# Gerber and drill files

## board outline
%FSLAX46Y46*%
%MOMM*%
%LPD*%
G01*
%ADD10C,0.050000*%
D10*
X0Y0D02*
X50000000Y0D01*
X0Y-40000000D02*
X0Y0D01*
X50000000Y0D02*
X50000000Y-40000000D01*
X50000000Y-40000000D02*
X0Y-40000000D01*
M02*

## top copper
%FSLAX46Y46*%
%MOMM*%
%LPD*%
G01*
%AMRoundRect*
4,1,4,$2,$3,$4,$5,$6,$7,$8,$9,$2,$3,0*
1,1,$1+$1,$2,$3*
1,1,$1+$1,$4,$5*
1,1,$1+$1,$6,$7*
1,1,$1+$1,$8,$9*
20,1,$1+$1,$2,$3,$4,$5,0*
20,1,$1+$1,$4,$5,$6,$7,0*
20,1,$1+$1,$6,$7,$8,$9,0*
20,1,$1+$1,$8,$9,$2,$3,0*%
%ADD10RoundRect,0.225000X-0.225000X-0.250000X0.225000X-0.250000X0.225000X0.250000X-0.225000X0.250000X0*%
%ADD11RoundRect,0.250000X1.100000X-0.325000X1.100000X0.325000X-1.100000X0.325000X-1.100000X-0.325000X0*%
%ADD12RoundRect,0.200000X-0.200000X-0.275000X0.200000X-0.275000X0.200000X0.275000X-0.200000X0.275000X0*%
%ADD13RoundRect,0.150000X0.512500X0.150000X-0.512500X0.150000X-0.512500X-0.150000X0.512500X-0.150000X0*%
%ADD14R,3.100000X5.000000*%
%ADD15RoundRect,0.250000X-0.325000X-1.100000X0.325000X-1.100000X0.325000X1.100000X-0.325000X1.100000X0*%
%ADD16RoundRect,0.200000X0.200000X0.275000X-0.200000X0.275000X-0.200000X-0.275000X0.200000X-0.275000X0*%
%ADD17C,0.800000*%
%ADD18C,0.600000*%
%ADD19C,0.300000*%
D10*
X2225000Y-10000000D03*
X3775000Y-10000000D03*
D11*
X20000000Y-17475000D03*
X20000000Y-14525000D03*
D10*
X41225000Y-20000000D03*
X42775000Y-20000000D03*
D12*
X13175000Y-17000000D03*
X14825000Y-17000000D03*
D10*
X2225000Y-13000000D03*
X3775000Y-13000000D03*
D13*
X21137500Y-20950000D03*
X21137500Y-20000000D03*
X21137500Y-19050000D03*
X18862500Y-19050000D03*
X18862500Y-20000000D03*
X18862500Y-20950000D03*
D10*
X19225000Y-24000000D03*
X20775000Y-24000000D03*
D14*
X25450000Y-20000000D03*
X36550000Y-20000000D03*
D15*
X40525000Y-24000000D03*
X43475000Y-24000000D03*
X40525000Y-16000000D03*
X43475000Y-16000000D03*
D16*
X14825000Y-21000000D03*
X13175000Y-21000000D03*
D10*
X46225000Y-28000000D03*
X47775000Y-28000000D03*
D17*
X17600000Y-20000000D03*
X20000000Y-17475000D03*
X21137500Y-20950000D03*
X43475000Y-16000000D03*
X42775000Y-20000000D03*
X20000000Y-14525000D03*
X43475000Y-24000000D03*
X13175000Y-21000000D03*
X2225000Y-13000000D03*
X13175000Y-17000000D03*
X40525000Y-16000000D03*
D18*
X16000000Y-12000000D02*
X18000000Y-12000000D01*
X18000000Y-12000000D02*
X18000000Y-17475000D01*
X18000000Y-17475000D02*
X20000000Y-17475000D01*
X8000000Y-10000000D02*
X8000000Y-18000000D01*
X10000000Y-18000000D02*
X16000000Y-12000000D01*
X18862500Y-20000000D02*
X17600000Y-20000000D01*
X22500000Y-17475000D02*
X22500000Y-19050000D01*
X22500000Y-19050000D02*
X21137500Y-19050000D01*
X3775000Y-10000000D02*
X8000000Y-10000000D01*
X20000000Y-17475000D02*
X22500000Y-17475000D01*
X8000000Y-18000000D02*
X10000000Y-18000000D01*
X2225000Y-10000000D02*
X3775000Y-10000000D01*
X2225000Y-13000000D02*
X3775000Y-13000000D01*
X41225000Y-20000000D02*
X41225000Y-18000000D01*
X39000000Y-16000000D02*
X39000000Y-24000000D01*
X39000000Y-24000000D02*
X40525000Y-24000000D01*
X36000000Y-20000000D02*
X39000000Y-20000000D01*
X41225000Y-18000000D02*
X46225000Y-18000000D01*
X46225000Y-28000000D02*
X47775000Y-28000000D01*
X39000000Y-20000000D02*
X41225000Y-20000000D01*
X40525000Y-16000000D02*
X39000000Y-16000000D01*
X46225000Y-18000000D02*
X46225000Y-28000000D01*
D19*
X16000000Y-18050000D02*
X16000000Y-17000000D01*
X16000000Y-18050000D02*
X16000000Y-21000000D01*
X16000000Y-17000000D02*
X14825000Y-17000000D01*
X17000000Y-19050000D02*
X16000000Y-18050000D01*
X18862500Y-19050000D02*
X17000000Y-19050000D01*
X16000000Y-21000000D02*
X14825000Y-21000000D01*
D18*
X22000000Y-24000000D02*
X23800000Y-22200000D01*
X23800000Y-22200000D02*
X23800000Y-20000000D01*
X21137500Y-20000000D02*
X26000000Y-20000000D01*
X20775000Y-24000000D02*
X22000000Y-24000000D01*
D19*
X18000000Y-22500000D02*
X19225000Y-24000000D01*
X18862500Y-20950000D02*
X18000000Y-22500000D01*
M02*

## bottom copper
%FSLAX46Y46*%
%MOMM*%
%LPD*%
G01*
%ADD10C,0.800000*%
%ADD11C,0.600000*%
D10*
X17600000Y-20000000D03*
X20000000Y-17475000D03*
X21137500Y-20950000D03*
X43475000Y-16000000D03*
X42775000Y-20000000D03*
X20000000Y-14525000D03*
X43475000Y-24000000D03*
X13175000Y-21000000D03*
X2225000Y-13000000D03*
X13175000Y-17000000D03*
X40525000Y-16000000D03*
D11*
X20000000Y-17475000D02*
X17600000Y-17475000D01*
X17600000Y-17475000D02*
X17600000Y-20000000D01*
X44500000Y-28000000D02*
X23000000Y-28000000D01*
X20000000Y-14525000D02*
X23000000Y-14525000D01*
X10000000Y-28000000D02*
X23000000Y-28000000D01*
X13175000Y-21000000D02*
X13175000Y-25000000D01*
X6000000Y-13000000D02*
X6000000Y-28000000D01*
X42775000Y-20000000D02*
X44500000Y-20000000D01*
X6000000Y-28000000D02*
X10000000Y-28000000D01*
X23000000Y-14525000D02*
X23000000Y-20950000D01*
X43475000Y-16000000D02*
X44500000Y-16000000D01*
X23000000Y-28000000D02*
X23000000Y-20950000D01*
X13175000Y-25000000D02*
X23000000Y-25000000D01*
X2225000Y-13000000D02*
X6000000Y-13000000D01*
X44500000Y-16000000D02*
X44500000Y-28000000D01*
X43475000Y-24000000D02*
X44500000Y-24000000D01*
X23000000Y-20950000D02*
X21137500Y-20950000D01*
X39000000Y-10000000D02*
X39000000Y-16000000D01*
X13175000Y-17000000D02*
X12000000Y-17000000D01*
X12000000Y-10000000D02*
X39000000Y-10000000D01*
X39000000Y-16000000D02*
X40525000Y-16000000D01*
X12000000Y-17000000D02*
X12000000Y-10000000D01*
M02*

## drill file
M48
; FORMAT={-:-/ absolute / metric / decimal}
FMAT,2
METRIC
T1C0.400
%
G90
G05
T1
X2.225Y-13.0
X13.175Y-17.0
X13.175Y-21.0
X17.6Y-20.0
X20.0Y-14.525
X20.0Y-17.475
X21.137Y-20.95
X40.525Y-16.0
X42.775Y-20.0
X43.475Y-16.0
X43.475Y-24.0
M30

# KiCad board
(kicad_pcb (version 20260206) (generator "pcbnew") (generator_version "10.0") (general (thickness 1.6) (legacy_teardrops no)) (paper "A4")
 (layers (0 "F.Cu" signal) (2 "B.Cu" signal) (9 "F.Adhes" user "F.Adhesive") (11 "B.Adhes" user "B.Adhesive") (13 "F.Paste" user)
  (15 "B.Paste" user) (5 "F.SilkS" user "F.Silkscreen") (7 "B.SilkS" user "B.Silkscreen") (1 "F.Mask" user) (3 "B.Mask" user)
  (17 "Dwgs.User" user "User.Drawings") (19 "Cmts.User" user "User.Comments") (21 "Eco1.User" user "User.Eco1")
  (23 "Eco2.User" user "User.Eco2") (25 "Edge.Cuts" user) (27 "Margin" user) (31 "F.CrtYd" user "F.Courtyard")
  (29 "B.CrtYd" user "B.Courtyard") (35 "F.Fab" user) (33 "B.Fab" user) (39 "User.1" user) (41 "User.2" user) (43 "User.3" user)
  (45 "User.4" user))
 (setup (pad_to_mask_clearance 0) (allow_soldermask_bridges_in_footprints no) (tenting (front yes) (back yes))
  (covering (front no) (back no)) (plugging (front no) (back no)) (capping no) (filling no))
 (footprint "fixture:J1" (layer "F.Cu") (at 3 10)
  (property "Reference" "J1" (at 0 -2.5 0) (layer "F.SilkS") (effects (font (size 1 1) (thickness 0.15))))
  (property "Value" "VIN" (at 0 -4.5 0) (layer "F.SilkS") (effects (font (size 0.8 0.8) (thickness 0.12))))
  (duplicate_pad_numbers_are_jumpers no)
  (pad "1" smd roundrect (at -0.775 0) (size 0.9 0.95) (layers "F.Cu" "F.Mask" "F.Paste") (roundrect_rratio 0.25) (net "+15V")
   (thermal_bridge_angle 45))
  (pad "2" smd roundrect (at 0.775 0) (size 0.9 0.95) (layers "F.Cu" "F.Mask" "F.Paste") (roundrect_rratio 0.25) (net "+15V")
   (thermal_bridge_angle 45)))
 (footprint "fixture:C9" (layer "F.Cu") (at 20 16 90)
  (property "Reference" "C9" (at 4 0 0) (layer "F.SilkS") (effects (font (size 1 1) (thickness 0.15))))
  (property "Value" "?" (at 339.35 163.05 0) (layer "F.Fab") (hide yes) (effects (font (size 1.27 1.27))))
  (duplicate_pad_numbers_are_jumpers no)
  (pad "1" smd roundrect (at -1.475 0 90) (size 1.15 2.7) (layers "F.Cu" "F.Mask" "F.Paste") (roundrect_rratio 0.217391) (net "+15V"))
  (pad "2" smd roundrect (at 1.475 0 90) (size 1.15 2.7) (layers "F.Cu" "F.Mask" "F.Paste") (roundrect_rratio 0.217391) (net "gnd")))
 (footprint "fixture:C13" (layer "F.Cu") (at 42 20)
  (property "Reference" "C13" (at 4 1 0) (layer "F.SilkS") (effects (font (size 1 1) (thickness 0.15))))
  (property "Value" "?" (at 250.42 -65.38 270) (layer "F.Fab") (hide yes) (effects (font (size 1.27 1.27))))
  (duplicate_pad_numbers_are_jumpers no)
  (pad "1" smd roundrect (at -0.775 0) (size 0.9 0.95) (layers "F.Cu" "F.Mask" "F.Paste") (roundrect_rratio 0.25) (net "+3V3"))
  (pad "2" smd roundrect (at 0.775 0) (size 0.9 0.95) (layers "F.Cu" "F.Mask" "F.Paste") (roundrect_rratio 0.25) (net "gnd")))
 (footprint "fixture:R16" (layer "F.Cu") (at 14 17)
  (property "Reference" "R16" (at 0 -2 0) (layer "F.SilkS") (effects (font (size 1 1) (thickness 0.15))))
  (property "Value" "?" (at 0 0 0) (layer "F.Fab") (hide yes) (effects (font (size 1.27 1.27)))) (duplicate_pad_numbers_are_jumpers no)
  (pad "1" smd roundrect (at -0.825 0) (size 0.8 0.95) (layers "F.Cu" "F.Mask" "F.Paste") (roundrect_rratio 0.25) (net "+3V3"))
  (pad "2" smd roundrect (at 0.825 0) (size 0.8 0.95) (layers "F.Cu" "F.Mask" "F.Paste") (roundrect_rratio 0.25) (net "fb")))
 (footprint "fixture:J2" (layer "F.Cu") (at 3 13)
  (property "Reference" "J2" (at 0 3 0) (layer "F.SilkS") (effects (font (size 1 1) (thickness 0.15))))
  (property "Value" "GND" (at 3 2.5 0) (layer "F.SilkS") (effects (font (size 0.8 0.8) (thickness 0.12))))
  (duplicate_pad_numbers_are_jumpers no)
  (pad "1" smd roundrect (at -0.775 0) (size 0.9 0.95) (layers "F.Cu" "F.Mask" "F.Paste") (roundrect_rratio 0.25) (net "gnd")
   (thermal_bridge_angle 45))
  (pad "2" smd roundrect (at 0.775 0) (size 0.9 0.95) (layers "F.Cu" "F.Mask" "F.Paste") (roundrect_rratio 0.25) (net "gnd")
   (thermal_bridge_angle 45)))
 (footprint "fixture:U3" (layer "F.Cu") (at 20 20 180)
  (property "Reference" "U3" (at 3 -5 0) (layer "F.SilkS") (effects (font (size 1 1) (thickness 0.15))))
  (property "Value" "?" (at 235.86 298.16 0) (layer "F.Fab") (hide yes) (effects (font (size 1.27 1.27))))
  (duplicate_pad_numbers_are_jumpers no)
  (pad "1" smd roundrect (at -1.1375 -0.95 180) (size 1.325 0.6) (layers "F.Cu" "F.Mask" "F.Paste") (roundrect_rratio 0.25) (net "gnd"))
  (pad "2" smd roundrect (at -1.1375 0 180) (size 1.325 0.6) (layers "F.Cu" "F.Mask" "F.Paste") (roundrect_rratio 0.25) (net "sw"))
  (pad "3" smd roundrect (at -1.1375 0.95 180) (size 1.325 0.6) (layers "F.Cu" "F.Mask" "F.Paste") (roundrect_rratio 0.25) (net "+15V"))
  (pad "4" smd roundrect (at 1.1375 0.95 180) (size 1.325 0.6) (layers "F.Cu" "F.Mask" "F.Paste") (roundrect_rratio 0.25) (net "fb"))
  (pad "5" smd roundrect (at 1.1375 0 180) (size 1.325 0.6) (layers "F.Cu" "F.Mask" "F.Paste") (roundrect_rratio 0.25) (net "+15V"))
  (pad "6" smd roundrect (at 1.1375 -0.95 180) (size 1.325 0.6) (layers "F.Cu" "F.Mask" "F.Paste") (roundrect_rratio 0.25) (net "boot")))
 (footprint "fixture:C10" (layer "F.Cu") (at 20 24)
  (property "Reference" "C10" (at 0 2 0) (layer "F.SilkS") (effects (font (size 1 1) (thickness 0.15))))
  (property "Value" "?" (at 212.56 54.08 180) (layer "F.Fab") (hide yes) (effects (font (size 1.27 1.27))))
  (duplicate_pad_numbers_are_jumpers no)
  (pad "1" smd roundrect (at -0.775 0) (size 0.9 0.95) (layers "F.Cu" "F.Mask" "F.Paste") (roundrect_rratio 0.25) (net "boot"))
  (pad "2" smd roundrect (at 0.775 0) (size 0.9 0.95) (layers "F.Cu" "F.Mask" "F.Paste") (roundrect_rratio 0.25) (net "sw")))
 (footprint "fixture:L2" (layer "F.Cu") (at 31 20)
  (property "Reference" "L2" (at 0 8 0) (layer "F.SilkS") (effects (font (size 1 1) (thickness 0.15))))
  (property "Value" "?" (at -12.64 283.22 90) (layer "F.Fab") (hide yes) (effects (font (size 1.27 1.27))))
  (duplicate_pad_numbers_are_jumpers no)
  (pad "1" smd rect (at -5.55 0) (size 3.1 5) (layers "F.Cu" "F.Mask" "F.Paste") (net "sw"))
  (pad "2" smd rect (at 5.55 0) (size 3.1 5) (layers "F.Cu" "F.Mask" "F.Paste") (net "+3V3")))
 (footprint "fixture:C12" (layer "F.Cu") (at 42 24)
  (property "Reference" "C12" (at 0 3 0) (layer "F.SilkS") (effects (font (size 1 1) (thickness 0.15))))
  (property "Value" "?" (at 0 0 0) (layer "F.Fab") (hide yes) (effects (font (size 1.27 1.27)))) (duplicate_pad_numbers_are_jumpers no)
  (pad "1" smd roundrect (at -1.475 0) (size 1.15 2.7) (layers "F.Cu" "F.Mask" "F.Paste") (roundrect_rratio 0.217391) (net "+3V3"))
  (pad "2" smd roundrect (at 1.475 0) (size 1.15 2.7) (layers "F.Cu" "F.Mask" "F.Paste") (roundrect_rratio 0.217391) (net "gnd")))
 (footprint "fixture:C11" (layer "F.Cu") (at 42 16)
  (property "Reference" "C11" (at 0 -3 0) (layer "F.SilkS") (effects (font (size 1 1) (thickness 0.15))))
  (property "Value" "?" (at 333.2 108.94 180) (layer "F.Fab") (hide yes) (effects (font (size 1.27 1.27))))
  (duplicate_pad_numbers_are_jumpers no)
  (pad "1" smd roundrect (at -1.475 0) (size 1.15 2.7) (layers "F.Cu" "F.Mask" "F.Paste") (roundrect_rratio 0.217391) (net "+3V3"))
  (pad "2" smd roundrect (at 1.475 0) (size 1.15 2.7) (layers "F.Cu" "F.Mask" "F.Paste") (roundrect_rratio 0.217391) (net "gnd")))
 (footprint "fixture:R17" (layer "F.Cu") (at 14 21 180)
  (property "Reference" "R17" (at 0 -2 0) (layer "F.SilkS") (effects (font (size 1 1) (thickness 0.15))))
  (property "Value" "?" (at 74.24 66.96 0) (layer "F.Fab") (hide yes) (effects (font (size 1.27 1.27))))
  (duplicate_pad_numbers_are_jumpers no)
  (pad "1" smd roundrect (at -0.825 0 180) (size 0.8 0.95) (layers "F.Cu" "F.Mask" "F.Paste") (roundrect_rratio 0.25) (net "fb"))
  (pad "2" smd roundrect (at 0.825 0 180) (size 0.8 0.95) (layers "F.Cu" "F.Mask" "F.Paste") (roundrect_rratio 0.25) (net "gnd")))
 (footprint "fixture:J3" (layer "F.Cu") (at 47 28)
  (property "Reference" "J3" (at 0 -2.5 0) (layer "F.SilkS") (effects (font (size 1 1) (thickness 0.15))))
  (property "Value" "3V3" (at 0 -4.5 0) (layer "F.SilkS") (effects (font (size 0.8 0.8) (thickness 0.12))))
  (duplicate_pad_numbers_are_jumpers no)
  (pad "1" smd roundrect (at -0.775 0) (size 0.9 0.95) (layers "F.Cu" "F.Mask" "F.Paste") (roundrect_rratio 0.25) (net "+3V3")
   (thermal_bridge_angle 45))
  (pad "2" smd roundrect (at 0.775 0) (size 0.9 0.95) (layers "F.Cu" "F.Mask" "F.Paste") (roundrect_rratio 0.25) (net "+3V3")
   (thermal_bridge_angle 45)))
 (gr_line (start 0 0) (end 50 0) (stroke (width 0.05) (type default)) (layer "Edge.Cuts"))
 (gr_line (start 0 40) (end 0 0) (stroke (width 0.05) (type default)) (layer "Edge.Cuts"))
 (gr_line (start 50 0) (end 50 40) (stroke (width 0.05) (type default)) (layer "Edge.Cuts"))
 (gr_line (start 50 40) (end 0 40) (stroke (width 0.05) (type default)) (layer "Edge.Cuts"))
 (segment (start 16 12) (end 18 12) (width 0.6) (layer "F.Cu") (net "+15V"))
 (segment (start 18 12) (end 18 17.475) (width 0.6) (layer "F.Cu") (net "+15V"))
 (segment (start 18 17.475) (end 20 17.475) (width 0.6) (layer "F.Cu") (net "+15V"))
 (segment (start 8 10) (end 8 18) (width 0.6) (layer "F.Cu") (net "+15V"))
 (segment (start 10 18) (end 16 12) (width 0.6) (layer "F.Cu") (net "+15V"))
 (segment (start 18.8625 20) (end 17.6 20) (width 0.6) (layer "F.Cu") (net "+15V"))
 (segment (start 22.5 17.475) (end 22.5 19.05) (width 0.6) (layer "F.Cu") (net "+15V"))
 (segment (start 22.5 19.05) (end 21.1375 19.05) (width 0.6) (layer "F.Cu") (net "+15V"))
 (segment (start 3.775 10) (end 8 10) (width 0.6) (layer "F.Cu") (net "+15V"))
 (segment (start 20 17.475) (end 22.5 17.475) (width 0.6) (layer "F.Cu") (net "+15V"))
 (segment (start 8 18) (end 10 18) (width 0.6) (layer "F.Cu") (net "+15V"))
 (segment (start 2.225 10) (end 3.775 10) (width 0.6) (layer "F.Cu") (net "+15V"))
 (via (at 17.6 20) (size 0.8) (drill 0.4) (layers "F.Cu" "B.Cu") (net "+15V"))
 (via (at 20 17.475) (size 0.8) (drill 0.4) (layers "F.Cu" "B.Cu") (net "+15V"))
 (segment (start 20 17.475) (end 17.6 17.475) (width 0.6) (layer "B.Cu") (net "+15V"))
 (segment (start 17.6 17.475) (end 17.6 20) (width 0.6) (layer "B.Cu") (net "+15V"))
 (segment (start 2.225 13) (end 3.775 13) (width 0.6) (layer "F.Cu") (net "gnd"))
 (via (at 21.1375 20.95) (size 0.8) (drill 0.4) (layers "F.Cu" "B.Cu") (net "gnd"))
 (via (at 43.475 16) (size 0.8) (drill 0.4) (layers "F.Cu" "B.Cu") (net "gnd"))
 (via (at 42.775 20) (size 0.8) (drill 0.4) (layers "F.Cu" "B.Cu") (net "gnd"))
 (via (at 20 14.525) (size 0.8) (drill 0.4) (layers "F.Cu" "B.Cu") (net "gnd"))
 (via (at 43.475 24) (size 0.8) (drill 0.4) (layers "F.Cu" "B.Cu") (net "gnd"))
 (via (at 13.175 21) (size 0.8) (drill 0.4) (layers "F.Cu" "B.Cu") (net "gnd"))
 (via (at 2.225 13) (size 0.8) (drill 0.4) (layers "F.Cu" "B.Cu") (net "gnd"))
 (segment (start 44.5 28) (end 23 28) (width 0.6) (layer "B.Cu") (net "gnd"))
 (segment (start 20 14.525) (end 23 14.525) (width 0.6) (layer "B.Cu") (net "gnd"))
 (segment (start 10 28) (end 23 28) (width 0.6) (layer "B.Cu") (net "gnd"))
 (segment (start 13.175 21) (end 13.175 25) (width 0.6) (layer "B.Cu") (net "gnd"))
 (segment (start 6 13) (end 6 28) (width 0.6) (layer "B.Cu") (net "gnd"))
 (segment (start 42.775 20) (end 44.5 20) (width 0.6) (layer "B.Cu") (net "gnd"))
 (segment (start 6 28) (end 10 28) (width 0.6) (layer "B.Cu") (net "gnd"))
 (segment (start 23 14.525) (end 23 20.95) (width 0.6) (layer "B.Cu") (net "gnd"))
 (segment (start 43.475 16) (end 44.5 16) (width 0.6) (layer "B.Cu") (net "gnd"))
 (segment (start 23 28) (end 23 20.95) (width 0.6) (layer "B.Cu") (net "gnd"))
 (segment (start 13.175 25) (end 23 25) (width 0.6) (layer "B.Cu") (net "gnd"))
 (segment (start 2.225 13) (end 6 13) (width 0.6) (layer "B.Cu") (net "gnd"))
 (segment (start 44.5 16) (end 44.5 28) (width 0.6) (layer "B.Cu") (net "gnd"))
 (segment (start 43.475 24) (end 44.5 24) (width 0.6) (layer "B.Cu") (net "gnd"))
 (segment (start 23 20.95) (end 21.1375 20.95) (width 0.6) (layer "B.Cu") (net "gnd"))
 (segment (start 41.225 20) (end 41.225 18) (width 0.6) (layer "F.Cu") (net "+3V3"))
 (segment (start 39 16) (end 39 24) (width 0.6) (layer "F.Cu") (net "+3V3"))
 (segment (start 39 24) (end 40.525 24) (width 0.6) (layer "F.Cu") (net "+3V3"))
 (segment (start 36 20) (end 39 20) (width 0.6) (layer "F.Cu") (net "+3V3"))
 (segment (start 41.225 18) (end 46.225 18) (width 0.6) (layer "F.Cu") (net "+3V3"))
 (segment (start 46.225 28) (end 47.775 28) (width 0.6) (layer "F.Cu") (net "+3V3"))
 (segment (start 39 20) (end 41.225 20) (width 0.6) (layer "F.Cu") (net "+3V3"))
 (segment (start 40.525 16) (end 39 16) (width 0.6) (layer "F.Cu") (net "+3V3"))
 (segment (start 46.225 18) (end 46.225 28) (width 0.6) (layer "F.Cu") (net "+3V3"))
 (via (at 13.175 17) (size 0.8) (drill 0.4) (layers "F.Cu" "B.Cu") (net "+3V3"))
 (via (at 40.525 16) (size 0.8) (drill 0.4) (layers "F.Cu" "B.Cu") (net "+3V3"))
 (segment (start 39 10) (end 39 16) (width 0.6) (layer "B.Cu") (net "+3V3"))
 (segment (start 13.175 17) (end 12 17) (width 0.6) (layer "B.Cu") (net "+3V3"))
 (segment (start 12 10) (end 39 10) (width 0.6) (layer "B.Cu") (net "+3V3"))
 (segment (start 39 16) (end 40.525 16) (width 0.6) (layer "B.Cu") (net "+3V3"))
 (segment (start 12 17) (end 12 10) (width 0.6) (layer "B.Cu") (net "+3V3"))
 (segment (start 16 18.05) (end 16 17) (width 0.3) (layer "F.Cu") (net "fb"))
 (segment (start 16 18.05) (end 16 21) (width 0.3) (layer "F.Cu") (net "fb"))
 (segment (start 16 17) (end 14.825 17) (width 0.3) (layer "F.Cu") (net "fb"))
 (segment (start 17 19.05) (end 16 18.05) (width 0.3) (layer "F.Cu") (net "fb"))
 (segment (start 18.8625 19.05) (end 17 19.05) (width 0.3) (layer "F.Cu") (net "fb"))
 (segment (start 16 21) (end 14.825 21) (width 0.3) (layer "F.Cu") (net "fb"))
 (segment (start 22 24) (end 23.8 22.2) (width 0.6) (layer "F.Cu") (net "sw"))
 (segment (start 23.8 22.2) (end 23.8 20) (width 0.6) (layer "F.Cu") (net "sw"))
 (segment (start 21.1375 20) (end 26 20) (width 0.6) (layer "F.Cu") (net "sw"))
 (segment (start 20.775 24) (end 22 24) (width 0.6) (layer "F.Cu") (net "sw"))
 (segment (start 18 22.5) (end 19.225 24) (width 0.3) (layer "F.Cu") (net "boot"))
 (segment (start 18.8625 20.95) (end 18 22.5) (width 0.3) (layer "F.Cu") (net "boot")))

